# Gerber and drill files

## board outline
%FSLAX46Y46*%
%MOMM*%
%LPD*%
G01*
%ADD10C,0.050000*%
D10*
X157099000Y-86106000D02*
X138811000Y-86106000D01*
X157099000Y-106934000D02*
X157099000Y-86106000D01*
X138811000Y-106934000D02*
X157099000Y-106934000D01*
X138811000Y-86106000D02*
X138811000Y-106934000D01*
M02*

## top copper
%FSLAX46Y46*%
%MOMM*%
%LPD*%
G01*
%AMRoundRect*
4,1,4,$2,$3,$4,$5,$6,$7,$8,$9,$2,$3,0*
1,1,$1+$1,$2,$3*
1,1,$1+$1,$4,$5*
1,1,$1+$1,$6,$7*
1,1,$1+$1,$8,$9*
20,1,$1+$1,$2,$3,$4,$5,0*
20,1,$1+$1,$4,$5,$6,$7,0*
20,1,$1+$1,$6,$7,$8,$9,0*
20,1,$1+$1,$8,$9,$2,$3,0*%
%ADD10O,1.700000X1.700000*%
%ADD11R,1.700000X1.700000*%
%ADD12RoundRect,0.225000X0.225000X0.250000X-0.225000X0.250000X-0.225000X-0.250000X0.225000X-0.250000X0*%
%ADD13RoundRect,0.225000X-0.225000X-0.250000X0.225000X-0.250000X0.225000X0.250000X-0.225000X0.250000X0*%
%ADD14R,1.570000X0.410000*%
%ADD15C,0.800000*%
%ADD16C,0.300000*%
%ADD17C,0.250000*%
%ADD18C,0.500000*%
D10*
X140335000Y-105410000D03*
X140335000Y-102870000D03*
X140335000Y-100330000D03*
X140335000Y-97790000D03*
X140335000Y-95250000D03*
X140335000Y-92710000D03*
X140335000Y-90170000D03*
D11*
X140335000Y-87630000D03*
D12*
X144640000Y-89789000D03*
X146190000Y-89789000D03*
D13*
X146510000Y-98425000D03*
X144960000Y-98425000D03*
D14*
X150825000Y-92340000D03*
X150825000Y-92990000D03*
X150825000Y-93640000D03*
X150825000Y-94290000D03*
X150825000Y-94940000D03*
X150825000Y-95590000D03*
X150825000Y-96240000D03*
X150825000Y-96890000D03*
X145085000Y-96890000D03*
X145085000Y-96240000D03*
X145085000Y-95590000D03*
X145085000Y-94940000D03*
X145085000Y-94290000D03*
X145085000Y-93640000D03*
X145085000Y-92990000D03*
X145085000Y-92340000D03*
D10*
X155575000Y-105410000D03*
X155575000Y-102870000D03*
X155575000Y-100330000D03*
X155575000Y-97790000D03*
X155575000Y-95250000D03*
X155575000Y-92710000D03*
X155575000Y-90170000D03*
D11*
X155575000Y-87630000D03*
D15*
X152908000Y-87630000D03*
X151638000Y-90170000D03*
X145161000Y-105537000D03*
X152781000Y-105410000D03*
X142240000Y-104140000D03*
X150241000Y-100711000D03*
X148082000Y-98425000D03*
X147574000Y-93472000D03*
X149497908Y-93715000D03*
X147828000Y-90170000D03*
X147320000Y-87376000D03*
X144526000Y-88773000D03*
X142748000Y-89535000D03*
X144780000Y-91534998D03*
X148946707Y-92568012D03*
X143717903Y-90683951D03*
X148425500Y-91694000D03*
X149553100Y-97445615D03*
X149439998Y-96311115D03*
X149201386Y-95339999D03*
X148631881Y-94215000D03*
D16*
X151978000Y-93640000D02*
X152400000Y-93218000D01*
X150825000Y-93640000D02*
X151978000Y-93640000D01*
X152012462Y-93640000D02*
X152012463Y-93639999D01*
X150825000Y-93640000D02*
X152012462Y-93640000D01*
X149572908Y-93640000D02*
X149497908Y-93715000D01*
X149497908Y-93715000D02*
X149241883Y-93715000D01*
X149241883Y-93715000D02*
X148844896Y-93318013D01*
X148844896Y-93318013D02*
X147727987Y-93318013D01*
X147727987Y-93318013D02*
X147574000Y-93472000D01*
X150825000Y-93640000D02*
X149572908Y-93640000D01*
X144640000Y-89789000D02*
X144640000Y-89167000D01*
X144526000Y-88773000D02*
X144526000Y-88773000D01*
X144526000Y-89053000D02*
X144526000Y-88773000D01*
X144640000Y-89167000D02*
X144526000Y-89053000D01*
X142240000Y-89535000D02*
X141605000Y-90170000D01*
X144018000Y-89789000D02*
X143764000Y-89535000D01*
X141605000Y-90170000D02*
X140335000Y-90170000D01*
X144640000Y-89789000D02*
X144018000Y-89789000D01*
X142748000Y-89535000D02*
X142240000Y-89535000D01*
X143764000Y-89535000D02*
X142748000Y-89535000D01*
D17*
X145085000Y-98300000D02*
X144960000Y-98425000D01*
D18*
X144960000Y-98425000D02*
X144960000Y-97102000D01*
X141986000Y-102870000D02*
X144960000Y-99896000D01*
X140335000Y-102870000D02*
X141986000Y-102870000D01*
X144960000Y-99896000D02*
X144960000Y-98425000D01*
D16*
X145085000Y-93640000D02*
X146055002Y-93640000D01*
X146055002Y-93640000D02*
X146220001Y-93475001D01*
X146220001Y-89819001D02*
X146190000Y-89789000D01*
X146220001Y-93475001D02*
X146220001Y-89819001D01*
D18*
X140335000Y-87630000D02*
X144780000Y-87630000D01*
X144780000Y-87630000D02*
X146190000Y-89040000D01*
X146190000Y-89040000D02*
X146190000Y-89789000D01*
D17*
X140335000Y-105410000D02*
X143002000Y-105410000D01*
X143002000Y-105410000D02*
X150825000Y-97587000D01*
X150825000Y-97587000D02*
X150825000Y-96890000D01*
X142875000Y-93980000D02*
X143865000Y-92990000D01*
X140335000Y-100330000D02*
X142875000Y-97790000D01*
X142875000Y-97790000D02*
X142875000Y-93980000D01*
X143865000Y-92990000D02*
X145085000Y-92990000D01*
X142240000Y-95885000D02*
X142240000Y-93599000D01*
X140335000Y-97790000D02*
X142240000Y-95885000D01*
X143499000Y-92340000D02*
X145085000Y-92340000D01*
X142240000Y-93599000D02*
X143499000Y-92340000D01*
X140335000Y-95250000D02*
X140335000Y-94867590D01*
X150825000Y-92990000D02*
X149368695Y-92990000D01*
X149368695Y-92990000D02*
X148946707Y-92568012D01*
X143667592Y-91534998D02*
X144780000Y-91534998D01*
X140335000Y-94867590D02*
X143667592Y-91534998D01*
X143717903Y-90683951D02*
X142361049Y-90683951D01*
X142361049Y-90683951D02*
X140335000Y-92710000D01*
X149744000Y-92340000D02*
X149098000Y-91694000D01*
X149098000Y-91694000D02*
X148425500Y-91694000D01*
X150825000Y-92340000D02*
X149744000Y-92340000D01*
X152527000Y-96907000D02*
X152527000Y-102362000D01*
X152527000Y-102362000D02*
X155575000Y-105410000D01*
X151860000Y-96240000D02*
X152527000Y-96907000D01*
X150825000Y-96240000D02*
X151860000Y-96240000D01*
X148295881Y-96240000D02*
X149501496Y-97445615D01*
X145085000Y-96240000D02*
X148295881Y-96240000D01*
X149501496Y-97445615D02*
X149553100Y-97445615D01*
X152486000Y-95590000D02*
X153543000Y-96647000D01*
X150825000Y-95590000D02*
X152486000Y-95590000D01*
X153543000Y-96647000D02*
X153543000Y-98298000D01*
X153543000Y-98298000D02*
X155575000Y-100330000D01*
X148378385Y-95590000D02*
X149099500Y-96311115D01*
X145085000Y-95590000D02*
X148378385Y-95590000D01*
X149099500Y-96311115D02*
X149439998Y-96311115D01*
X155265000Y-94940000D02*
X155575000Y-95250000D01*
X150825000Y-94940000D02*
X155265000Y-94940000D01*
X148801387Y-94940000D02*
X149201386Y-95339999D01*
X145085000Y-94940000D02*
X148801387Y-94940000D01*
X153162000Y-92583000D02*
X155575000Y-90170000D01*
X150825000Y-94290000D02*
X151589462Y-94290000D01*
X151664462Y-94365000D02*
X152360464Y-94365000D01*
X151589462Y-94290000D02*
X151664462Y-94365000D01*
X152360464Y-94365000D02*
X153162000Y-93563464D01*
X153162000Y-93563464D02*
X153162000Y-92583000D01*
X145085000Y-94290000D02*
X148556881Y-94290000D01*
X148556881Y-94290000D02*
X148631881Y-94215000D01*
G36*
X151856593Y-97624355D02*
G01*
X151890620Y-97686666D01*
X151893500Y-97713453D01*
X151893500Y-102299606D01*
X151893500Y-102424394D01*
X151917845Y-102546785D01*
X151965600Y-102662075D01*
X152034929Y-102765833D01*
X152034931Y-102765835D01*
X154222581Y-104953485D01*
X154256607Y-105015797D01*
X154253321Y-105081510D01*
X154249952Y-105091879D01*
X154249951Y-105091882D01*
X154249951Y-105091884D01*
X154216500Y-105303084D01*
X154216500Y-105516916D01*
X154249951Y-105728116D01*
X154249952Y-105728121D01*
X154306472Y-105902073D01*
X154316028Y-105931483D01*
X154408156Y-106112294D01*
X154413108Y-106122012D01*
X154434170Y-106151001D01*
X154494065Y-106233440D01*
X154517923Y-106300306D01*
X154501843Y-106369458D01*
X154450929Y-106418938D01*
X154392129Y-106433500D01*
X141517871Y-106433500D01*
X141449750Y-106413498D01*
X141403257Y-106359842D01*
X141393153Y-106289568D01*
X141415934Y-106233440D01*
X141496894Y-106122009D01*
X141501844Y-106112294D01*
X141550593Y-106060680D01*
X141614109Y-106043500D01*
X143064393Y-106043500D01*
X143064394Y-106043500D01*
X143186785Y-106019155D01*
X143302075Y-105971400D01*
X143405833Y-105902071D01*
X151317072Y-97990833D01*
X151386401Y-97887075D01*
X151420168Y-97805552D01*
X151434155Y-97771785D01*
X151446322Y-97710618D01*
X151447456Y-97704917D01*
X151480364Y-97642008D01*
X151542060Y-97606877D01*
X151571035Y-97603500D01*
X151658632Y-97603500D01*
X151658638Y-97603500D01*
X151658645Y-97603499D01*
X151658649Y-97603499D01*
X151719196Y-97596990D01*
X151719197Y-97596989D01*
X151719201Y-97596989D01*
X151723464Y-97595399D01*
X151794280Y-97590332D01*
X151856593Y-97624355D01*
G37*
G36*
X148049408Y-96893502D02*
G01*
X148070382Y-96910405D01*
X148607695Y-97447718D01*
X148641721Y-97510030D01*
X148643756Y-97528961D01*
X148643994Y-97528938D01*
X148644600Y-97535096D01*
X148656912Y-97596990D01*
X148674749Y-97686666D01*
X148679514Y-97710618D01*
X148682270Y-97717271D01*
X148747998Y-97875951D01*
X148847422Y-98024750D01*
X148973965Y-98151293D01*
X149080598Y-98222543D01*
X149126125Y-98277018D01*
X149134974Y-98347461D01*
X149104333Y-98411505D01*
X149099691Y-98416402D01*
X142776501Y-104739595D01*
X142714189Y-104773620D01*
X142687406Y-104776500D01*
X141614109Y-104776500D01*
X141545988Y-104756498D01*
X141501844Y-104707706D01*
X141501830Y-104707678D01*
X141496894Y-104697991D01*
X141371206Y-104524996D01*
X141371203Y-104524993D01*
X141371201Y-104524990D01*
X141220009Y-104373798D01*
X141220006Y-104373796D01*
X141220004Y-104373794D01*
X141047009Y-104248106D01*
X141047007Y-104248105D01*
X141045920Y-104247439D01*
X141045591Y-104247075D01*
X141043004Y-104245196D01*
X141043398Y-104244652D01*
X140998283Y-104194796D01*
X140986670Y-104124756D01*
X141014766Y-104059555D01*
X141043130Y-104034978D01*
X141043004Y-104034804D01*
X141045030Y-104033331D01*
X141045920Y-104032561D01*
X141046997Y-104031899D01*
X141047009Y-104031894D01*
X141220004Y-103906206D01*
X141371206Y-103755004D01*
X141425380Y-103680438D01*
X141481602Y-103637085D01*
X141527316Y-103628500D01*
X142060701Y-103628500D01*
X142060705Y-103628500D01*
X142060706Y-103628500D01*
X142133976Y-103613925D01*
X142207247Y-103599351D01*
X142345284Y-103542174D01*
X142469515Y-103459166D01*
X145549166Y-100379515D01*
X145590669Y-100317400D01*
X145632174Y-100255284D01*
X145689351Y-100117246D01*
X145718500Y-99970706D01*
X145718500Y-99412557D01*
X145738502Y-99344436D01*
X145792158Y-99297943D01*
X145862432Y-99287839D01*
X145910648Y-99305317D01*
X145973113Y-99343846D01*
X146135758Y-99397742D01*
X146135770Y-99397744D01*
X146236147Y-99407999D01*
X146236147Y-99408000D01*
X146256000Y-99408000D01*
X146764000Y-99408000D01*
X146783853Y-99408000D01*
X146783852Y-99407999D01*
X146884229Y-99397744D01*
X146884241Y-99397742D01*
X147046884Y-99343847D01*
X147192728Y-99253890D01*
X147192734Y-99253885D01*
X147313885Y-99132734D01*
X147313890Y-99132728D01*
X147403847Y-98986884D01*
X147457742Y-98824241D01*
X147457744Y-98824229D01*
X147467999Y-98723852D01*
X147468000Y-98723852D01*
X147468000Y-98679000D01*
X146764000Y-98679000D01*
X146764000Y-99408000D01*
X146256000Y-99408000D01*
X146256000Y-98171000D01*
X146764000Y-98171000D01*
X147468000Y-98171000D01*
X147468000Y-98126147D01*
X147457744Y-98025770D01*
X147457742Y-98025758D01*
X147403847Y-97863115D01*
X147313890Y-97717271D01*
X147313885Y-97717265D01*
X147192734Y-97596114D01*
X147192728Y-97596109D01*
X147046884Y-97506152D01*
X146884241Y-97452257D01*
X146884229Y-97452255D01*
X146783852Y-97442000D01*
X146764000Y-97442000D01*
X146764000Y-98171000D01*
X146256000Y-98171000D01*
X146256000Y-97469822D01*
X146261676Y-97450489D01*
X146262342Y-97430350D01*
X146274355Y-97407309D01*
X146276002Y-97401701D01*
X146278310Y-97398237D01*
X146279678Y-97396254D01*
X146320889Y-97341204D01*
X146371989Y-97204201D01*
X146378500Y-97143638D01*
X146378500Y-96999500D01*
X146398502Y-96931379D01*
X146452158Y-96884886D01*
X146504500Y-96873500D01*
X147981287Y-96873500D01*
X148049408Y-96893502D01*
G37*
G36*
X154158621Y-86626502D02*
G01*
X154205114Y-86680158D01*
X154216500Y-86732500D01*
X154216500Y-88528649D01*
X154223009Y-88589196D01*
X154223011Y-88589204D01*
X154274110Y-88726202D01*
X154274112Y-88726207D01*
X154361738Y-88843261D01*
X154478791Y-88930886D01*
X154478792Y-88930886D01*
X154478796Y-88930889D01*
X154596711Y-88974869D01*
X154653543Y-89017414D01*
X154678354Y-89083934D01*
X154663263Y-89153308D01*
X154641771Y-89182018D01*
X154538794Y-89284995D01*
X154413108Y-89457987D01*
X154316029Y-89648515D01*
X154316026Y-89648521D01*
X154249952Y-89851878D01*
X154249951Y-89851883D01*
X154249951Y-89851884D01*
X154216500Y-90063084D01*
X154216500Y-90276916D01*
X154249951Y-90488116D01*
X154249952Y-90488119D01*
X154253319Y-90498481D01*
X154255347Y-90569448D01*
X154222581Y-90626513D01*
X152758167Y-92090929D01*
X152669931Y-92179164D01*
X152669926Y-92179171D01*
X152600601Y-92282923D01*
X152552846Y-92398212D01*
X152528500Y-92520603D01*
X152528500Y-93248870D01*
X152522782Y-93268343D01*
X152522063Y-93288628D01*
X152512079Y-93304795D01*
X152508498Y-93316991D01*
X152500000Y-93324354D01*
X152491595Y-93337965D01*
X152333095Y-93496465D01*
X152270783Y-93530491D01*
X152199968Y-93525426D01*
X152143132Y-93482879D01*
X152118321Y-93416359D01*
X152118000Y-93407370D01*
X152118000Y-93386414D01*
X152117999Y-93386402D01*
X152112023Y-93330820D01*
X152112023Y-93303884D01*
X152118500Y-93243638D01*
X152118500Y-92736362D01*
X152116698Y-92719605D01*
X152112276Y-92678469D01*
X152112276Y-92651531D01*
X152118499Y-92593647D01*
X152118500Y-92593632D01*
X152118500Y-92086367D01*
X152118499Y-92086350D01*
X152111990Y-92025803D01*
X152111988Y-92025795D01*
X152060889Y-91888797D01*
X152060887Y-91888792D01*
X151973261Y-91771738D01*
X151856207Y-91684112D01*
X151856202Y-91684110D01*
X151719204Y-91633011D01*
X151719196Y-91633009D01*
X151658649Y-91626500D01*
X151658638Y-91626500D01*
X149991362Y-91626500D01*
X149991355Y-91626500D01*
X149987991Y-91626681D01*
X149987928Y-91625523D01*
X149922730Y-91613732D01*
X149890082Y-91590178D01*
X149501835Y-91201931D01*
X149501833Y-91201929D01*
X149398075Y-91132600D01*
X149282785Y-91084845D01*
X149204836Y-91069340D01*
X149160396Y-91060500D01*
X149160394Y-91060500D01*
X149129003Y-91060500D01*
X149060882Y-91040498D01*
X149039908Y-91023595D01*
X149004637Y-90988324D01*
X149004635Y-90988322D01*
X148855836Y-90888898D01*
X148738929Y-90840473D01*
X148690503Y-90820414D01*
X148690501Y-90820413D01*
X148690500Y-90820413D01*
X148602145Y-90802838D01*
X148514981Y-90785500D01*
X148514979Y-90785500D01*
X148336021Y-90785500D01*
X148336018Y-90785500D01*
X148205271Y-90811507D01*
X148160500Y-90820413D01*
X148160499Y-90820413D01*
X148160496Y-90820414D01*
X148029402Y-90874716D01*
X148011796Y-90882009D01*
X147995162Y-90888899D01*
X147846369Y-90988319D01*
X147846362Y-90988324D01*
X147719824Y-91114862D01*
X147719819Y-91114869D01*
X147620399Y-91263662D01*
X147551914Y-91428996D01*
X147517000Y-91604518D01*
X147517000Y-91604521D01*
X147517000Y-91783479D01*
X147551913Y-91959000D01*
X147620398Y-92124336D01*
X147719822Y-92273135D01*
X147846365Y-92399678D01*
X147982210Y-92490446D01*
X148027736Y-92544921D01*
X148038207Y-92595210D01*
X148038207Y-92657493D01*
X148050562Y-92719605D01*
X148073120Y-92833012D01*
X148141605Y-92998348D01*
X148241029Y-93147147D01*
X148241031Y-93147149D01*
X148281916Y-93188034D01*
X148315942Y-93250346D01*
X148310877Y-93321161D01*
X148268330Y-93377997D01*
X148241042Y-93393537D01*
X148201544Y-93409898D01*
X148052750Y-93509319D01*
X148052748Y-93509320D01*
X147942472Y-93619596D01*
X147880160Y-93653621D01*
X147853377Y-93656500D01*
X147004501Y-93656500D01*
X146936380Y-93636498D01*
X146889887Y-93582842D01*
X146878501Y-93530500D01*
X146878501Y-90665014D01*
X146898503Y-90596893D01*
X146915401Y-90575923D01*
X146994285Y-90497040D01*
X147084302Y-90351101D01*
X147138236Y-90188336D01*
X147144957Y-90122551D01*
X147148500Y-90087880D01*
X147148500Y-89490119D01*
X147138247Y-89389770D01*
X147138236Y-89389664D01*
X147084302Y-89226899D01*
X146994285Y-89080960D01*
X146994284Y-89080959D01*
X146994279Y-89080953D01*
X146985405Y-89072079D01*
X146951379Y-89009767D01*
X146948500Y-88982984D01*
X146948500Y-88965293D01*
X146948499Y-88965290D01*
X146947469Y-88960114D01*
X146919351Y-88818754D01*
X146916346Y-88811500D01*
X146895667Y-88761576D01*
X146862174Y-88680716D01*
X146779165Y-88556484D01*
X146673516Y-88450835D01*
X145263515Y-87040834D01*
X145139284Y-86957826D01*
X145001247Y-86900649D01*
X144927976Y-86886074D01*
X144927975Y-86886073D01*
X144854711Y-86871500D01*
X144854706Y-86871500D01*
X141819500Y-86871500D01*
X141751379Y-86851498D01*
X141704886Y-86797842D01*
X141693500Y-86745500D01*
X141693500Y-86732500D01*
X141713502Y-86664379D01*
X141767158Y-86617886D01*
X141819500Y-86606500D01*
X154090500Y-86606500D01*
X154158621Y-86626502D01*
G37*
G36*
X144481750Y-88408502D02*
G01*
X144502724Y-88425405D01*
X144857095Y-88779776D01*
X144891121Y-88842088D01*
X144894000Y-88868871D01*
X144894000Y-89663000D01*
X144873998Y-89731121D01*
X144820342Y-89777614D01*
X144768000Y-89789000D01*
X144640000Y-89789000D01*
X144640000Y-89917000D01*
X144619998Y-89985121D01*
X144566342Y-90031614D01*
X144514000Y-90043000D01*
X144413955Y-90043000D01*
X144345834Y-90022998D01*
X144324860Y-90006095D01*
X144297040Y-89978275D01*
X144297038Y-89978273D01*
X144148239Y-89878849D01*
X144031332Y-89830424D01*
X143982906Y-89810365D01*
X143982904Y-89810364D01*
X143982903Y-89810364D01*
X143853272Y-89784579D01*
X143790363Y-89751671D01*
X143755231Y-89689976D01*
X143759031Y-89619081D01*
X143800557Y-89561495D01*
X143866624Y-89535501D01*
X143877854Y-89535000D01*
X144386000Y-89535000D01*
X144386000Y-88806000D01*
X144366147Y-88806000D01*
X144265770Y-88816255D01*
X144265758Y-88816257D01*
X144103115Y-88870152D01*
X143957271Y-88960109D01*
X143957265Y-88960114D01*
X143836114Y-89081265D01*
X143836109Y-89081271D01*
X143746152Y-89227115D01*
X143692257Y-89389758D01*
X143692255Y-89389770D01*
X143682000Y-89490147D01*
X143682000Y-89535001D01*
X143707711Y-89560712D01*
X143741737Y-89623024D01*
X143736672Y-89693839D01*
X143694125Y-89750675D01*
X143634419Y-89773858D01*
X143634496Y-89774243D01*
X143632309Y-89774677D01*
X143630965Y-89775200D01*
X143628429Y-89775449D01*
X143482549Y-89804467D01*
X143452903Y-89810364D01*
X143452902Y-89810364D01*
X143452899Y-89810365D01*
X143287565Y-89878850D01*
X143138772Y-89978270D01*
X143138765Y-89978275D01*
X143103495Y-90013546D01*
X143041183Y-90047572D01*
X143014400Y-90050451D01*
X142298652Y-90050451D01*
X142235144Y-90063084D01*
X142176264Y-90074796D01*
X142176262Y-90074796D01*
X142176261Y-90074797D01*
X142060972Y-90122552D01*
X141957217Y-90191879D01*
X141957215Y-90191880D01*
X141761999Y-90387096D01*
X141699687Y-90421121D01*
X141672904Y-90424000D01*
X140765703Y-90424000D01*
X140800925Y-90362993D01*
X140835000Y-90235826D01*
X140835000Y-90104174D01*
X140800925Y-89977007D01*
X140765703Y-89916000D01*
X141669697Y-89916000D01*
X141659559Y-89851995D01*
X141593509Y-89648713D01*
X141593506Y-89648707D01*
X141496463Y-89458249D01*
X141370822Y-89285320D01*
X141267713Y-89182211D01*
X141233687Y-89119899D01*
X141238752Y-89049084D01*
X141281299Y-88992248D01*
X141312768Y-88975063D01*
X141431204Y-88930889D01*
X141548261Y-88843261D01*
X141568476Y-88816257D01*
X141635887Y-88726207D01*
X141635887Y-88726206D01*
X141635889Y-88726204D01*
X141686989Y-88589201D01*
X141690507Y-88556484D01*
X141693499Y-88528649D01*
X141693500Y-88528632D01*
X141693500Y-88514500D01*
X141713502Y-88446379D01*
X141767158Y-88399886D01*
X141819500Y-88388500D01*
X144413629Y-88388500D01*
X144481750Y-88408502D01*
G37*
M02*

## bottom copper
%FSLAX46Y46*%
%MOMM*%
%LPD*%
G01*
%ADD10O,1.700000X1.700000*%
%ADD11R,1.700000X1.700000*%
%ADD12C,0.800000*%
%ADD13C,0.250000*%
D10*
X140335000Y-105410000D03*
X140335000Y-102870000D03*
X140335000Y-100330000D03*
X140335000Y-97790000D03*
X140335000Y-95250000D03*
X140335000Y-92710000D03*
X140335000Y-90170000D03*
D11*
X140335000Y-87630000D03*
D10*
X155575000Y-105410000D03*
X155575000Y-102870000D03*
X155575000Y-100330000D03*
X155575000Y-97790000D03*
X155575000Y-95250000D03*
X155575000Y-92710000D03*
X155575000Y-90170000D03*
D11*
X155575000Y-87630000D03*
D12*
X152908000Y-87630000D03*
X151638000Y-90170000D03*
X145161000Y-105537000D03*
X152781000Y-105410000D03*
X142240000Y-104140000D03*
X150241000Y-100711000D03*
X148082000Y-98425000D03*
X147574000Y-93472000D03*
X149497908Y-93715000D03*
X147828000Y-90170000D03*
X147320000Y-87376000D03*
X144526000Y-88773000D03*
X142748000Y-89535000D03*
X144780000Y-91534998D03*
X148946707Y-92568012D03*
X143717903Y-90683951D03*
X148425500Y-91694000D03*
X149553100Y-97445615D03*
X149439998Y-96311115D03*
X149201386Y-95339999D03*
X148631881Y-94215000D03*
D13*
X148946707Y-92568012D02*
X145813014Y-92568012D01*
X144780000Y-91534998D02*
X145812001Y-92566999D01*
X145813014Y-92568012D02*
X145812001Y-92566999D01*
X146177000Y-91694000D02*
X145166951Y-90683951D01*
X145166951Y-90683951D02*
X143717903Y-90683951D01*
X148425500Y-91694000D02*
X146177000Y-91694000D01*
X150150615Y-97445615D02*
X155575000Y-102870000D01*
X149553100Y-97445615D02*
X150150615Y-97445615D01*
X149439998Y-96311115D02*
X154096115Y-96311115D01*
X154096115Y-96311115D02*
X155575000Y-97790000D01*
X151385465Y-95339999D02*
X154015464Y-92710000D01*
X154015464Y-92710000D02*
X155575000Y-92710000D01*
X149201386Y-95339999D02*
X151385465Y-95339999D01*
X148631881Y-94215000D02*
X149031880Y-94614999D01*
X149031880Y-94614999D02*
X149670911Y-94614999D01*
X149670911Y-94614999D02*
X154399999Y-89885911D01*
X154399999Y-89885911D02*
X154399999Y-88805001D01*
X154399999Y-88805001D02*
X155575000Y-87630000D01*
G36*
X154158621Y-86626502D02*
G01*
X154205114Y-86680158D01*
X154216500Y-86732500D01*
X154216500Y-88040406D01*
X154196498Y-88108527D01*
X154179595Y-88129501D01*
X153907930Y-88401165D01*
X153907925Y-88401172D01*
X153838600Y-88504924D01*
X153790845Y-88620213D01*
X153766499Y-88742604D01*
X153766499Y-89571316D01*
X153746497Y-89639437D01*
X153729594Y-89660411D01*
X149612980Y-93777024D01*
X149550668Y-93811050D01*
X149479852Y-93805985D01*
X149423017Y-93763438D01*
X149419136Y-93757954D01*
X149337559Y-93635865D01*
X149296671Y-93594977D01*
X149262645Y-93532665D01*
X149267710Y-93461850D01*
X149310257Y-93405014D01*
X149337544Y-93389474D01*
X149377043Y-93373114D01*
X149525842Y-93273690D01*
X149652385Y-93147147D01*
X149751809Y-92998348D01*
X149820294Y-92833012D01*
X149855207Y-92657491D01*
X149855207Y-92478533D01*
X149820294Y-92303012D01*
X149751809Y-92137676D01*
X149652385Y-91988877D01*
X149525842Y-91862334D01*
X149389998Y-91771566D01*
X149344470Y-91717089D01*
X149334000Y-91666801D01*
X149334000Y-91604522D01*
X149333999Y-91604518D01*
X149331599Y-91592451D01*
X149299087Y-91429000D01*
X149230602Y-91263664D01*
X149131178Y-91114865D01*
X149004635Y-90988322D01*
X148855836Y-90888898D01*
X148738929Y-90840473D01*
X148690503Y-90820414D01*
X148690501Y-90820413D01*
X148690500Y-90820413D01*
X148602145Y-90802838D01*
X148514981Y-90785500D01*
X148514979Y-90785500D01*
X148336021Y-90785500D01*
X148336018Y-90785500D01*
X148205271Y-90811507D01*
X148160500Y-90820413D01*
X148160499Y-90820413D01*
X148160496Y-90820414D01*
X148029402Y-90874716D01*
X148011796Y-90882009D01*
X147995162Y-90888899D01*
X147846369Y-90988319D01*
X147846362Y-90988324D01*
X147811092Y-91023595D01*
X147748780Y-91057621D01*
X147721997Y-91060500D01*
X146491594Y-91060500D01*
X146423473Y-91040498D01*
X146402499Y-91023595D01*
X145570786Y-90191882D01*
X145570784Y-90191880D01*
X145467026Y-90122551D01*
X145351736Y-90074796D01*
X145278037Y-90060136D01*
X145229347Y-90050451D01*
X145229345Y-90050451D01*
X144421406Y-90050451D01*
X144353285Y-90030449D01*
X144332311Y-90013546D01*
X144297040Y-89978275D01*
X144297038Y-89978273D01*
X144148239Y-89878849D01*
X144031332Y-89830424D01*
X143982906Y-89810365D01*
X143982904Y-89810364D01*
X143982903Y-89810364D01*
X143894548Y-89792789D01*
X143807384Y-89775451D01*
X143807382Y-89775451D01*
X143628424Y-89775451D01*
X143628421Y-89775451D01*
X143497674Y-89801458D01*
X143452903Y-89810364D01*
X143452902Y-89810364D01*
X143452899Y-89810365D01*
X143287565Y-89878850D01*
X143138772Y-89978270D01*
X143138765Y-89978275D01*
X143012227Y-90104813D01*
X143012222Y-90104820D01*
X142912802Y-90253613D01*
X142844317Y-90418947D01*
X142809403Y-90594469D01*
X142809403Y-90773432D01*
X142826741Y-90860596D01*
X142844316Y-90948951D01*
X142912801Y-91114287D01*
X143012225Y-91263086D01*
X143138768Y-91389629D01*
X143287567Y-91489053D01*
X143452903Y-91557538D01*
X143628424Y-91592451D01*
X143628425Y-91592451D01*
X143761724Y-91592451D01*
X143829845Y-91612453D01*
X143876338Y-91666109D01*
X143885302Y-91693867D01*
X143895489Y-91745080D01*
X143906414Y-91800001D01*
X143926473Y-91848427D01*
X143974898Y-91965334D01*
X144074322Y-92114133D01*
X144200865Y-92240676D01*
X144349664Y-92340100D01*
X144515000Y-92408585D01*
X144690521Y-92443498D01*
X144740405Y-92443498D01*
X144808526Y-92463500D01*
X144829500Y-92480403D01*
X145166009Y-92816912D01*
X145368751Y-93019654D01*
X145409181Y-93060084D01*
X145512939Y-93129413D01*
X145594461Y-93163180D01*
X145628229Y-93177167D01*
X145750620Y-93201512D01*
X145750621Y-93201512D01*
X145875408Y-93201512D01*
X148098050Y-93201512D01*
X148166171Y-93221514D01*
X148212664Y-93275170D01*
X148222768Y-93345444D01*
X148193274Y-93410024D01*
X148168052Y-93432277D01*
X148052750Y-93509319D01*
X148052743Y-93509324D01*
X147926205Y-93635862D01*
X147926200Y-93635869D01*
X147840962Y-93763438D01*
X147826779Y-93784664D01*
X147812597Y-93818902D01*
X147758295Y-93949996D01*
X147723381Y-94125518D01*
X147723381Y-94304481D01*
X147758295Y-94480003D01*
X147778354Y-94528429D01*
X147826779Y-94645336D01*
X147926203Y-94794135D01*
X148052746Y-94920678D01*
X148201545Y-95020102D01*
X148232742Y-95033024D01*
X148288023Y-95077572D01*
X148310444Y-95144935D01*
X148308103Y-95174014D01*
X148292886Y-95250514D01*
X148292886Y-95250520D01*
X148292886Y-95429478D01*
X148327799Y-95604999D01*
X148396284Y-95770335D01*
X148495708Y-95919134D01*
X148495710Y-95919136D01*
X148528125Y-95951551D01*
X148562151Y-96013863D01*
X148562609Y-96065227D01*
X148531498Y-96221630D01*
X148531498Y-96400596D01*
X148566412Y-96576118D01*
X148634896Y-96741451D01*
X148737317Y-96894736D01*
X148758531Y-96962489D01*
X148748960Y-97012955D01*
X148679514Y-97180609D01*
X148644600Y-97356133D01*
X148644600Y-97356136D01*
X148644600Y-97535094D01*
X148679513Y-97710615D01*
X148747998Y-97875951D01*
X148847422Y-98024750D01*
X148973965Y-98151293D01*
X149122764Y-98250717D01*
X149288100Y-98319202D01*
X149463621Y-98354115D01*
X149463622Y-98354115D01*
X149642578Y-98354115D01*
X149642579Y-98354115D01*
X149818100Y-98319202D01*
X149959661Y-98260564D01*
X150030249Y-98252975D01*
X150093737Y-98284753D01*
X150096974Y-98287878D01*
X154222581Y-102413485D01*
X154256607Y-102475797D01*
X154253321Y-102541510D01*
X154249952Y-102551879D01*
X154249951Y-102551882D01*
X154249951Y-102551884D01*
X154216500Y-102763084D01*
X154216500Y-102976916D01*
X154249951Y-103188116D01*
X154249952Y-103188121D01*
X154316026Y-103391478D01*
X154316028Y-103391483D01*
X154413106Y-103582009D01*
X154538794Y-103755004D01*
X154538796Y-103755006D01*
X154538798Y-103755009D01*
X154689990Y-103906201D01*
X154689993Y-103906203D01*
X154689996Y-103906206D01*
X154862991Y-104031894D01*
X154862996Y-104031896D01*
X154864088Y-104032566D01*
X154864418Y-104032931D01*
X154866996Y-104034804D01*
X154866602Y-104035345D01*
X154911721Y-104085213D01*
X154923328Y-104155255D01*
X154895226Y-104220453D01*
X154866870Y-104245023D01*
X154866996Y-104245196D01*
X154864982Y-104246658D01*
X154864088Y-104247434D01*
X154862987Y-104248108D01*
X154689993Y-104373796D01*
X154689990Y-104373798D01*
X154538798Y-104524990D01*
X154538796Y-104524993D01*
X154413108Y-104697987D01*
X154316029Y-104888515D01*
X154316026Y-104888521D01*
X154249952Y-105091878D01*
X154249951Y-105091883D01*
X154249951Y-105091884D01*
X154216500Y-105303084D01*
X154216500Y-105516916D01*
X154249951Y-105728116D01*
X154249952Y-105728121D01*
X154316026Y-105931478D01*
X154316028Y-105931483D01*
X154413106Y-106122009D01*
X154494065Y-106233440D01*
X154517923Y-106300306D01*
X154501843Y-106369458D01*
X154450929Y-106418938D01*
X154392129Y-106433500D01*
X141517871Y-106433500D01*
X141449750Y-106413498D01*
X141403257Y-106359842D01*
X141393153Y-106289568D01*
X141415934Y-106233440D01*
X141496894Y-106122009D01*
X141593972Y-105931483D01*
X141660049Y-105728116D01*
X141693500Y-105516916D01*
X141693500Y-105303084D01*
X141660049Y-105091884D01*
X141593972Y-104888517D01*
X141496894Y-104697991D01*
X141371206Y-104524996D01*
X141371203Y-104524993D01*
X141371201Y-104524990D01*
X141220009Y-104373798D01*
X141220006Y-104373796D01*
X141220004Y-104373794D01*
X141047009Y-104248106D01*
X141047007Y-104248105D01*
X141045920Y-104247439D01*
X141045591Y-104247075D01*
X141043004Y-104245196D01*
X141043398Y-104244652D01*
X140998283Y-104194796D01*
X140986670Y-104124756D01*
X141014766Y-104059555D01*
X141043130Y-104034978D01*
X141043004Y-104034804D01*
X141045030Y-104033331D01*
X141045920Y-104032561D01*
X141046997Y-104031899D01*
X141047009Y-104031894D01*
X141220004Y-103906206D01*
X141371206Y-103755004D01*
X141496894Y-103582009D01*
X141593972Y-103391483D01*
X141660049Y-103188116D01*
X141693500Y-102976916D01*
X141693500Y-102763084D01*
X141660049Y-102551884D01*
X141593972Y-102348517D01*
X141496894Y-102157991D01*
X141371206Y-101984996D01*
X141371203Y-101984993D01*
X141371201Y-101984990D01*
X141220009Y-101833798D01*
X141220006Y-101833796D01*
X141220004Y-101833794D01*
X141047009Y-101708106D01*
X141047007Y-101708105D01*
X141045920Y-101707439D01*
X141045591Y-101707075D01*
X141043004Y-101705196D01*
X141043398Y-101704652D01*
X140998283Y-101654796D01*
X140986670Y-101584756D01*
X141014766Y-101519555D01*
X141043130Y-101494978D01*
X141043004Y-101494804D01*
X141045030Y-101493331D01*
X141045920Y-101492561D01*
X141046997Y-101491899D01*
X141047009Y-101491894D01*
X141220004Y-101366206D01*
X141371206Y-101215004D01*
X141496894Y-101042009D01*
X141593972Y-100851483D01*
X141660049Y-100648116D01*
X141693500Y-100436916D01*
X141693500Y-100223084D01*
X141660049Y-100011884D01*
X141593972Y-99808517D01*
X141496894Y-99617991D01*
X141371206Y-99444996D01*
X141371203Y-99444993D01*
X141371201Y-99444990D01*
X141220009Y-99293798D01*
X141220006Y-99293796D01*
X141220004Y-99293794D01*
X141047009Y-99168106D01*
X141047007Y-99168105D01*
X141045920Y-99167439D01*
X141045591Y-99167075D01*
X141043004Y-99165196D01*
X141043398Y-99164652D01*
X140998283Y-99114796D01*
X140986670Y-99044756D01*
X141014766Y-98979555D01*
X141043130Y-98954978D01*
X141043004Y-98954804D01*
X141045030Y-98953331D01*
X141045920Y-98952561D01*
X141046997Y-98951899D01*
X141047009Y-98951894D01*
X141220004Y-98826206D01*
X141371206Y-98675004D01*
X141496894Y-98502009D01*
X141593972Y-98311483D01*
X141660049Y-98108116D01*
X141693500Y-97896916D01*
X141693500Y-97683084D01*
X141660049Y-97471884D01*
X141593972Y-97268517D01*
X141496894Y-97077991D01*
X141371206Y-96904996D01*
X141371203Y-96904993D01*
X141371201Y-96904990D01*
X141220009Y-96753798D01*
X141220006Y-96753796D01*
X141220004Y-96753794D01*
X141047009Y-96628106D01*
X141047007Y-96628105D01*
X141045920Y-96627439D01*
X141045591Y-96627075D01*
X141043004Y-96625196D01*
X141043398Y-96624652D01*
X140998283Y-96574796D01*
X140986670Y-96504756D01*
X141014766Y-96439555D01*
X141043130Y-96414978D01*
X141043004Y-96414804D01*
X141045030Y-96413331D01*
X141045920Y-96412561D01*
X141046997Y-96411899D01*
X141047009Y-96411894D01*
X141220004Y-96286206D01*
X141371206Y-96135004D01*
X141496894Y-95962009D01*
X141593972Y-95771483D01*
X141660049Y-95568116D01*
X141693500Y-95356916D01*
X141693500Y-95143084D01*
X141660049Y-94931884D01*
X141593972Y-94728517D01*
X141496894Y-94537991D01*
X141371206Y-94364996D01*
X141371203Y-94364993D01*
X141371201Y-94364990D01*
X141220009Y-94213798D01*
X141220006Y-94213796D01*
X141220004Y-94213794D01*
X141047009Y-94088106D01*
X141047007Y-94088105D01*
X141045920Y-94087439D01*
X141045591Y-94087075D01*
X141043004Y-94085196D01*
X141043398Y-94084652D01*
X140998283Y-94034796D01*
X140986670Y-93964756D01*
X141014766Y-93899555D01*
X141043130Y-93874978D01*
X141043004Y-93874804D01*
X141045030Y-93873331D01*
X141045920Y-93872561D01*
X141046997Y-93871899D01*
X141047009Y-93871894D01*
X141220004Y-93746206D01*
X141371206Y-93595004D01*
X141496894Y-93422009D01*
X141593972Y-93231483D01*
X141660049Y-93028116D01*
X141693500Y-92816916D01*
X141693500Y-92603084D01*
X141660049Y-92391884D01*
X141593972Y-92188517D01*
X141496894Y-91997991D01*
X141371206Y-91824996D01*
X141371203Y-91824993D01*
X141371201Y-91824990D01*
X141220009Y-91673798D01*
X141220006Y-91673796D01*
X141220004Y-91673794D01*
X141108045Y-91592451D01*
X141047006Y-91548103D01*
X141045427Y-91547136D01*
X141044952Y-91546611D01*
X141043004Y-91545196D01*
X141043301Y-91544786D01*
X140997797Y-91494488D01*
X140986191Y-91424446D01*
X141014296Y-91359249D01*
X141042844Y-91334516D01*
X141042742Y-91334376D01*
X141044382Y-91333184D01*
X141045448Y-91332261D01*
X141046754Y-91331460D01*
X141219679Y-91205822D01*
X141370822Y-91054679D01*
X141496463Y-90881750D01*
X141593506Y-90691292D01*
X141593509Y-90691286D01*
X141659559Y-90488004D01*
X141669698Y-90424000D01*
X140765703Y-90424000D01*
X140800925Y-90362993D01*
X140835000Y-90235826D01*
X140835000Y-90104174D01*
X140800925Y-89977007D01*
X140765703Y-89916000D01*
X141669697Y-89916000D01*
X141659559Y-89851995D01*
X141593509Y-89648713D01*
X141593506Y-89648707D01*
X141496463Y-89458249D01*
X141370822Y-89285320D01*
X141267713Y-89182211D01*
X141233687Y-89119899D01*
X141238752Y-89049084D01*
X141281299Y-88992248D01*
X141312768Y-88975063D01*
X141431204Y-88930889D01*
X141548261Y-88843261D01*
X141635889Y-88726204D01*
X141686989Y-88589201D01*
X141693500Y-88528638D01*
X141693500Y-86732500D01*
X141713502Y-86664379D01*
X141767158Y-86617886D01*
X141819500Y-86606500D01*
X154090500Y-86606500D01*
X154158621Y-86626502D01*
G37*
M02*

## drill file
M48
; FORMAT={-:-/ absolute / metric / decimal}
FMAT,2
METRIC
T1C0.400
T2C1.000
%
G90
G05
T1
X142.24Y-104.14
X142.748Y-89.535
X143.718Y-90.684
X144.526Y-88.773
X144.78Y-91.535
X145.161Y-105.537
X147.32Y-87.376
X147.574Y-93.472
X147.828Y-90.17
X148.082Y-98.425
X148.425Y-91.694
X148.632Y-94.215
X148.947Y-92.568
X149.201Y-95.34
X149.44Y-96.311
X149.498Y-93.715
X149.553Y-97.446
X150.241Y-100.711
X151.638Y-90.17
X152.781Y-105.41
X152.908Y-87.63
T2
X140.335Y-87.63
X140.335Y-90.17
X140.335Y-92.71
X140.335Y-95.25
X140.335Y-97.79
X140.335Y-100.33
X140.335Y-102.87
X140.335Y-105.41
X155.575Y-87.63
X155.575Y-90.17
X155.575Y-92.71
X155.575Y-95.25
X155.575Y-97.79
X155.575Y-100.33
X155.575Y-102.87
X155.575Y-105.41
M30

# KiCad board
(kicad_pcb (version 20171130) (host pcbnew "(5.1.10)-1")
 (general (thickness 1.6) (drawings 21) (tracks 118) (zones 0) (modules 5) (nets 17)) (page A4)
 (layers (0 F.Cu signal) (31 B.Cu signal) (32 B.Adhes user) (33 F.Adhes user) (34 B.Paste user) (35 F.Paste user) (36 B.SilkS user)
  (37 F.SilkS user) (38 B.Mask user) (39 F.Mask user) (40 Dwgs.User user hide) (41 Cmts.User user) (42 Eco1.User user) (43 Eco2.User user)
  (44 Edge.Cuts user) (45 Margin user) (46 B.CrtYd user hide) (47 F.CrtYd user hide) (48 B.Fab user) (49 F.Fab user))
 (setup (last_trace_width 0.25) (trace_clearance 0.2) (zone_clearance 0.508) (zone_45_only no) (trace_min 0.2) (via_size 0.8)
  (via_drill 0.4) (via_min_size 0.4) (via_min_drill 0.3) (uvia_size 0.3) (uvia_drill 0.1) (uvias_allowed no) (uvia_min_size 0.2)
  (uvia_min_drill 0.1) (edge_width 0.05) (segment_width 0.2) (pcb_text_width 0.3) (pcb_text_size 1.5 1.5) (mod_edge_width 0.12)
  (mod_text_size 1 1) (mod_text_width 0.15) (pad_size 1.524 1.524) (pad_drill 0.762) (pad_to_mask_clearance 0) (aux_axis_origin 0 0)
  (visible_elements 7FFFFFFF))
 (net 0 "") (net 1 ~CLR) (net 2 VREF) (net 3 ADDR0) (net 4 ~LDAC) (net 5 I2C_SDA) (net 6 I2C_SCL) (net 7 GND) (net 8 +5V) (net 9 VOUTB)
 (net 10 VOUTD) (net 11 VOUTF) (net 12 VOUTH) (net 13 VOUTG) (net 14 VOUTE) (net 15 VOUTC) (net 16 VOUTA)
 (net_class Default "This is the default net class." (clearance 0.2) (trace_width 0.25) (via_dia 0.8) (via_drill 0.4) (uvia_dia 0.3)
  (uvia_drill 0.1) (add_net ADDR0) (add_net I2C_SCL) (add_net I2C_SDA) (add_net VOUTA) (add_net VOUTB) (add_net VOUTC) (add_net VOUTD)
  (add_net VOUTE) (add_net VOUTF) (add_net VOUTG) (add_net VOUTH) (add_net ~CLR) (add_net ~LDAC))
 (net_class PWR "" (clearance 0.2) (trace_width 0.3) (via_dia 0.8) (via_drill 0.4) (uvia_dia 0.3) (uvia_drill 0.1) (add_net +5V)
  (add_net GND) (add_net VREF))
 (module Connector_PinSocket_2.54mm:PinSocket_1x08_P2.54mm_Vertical (layer B.Cu) (at 140.335 87.63 180)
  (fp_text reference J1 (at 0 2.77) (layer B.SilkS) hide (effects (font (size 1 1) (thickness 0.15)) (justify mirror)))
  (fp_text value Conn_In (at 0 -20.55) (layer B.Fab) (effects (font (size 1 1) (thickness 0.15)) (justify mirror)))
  (pad 8 thru_hole oval (at 0 -17.78 180) (size 1.7 1.7) (drill 1) (layers *.Cu *.Mask) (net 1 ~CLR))
  (pad 7 thru_hole oval (at 0 -15.24 180) (size 1.7 1.7) (drill 1) (layers *.Cu *.Mask) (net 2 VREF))
  (pad 6 thru_hole oval (at 0 -12.7 180) (size 1.7 1.7) (drill 1) (layers *.Cu *.Mask) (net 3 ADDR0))
  (pad 5 thru_hole oval (at 0 -10.16 180) (size 1.7 1.7) (drill 1) (layers *.Cu *.Mask) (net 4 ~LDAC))
  (pad 4 thru_hole oval (at 0 -7.62 180) (size 1.7 1.7) (drill 1) (layers *.Cu *.Mask) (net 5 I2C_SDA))
  (pad 3 thru_hole oval (at 0 -5.08 180) (size 1.7 1.7) (drill 1) (layers *.Cu *.Mask) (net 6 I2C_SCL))
  (pad 2 thru_hole oval (at 0 -2.54 180) (size 1.7 1.7) (drill 1) (layers *.Cu *.Mask) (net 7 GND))
  (pad 1 thru_hole rect (at 0 0 180) (size 1.7 1.7) (drill 1) (layers *.Cu *.Mask) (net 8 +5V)))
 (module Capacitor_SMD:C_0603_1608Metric (layer F.Cu) (at 145.415 89.789 180)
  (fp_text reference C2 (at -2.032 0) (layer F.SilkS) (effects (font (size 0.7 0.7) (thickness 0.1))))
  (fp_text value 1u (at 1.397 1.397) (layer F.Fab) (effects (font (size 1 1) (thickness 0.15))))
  (pad 2 smd roundrect (at 0.775 0 180) (size 0.9 0.95) (layers F.Cu F.Paste F.Mask) (roundrect_rratio 0.25) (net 7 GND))
  (pad 1 smd roundrect (at -0.775 0 180) (size 0.9 0.95) (layers F.Cu F.Paste F.Mask) (roundrect_rratio 0.25) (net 8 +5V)))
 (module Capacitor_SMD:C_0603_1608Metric (layer F.Cu) (at 145.735 98.425)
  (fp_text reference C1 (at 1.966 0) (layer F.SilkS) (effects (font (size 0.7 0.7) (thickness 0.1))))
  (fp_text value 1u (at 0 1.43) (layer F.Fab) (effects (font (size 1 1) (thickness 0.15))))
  (pad 2 smd roundrect (at 0.775 0) (size 0.9 0.95) (layers F.Cu F.Paste F.Mask) (roundrect_rratio 0.25) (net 7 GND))
  (pad 1 smd roundrect (at -0.775 0) (size 0.9 0.95) (layers F.Cu F.Paste F.Mask) (roundrect_rratio 0.25) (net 2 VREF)))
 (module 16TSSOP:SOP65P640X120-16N (layer F.Cu) (at 147.955 94.615)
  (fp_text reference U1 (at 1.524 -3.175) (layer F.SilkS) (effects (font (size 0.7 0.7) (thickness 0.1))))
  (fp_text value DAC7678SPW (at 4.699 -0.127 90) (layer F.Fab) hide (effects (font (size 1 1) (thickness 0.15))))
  (pad 16 smd rect (at 2.87 -2.275) (size 1.57 0.41) (layers F.Cu F.Paste F.Mask) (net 6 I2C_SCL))
  (pad 15 smd rect (at 2.87 -1.625) (size 1.57 0.41) (layers F.Cu F.Paste F.Mask) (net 5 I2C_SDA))
  (pad 14 smd rect (at 2.87 -0.975) (size 1.57 0.41) (layers F.Cu F.Paste F.Mask) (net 7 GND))
  (pad 13 smd rect (at 2.87 -0.325) (size 1.57 0.41) (layers F.Cu F.Paste F.Mask) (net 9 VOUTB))
  (pad 12 smd rect (at 2.87 0.325) (size 1.57 0.41) (layers F.Cu F.Paste F.Mask) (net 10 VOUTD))
  (pad 11 smd rect (at 2.87 0.975) (size 1.57 0.41) (layers F.Cu F.Paste F.Mask) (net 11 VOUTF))
  (pad 10 smd rect (at 2.87 1.625) (size 1.57 0.41) (layers F.Cu F.Paste F.Mask) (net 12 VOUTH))
  (pad 9 smd rect (at 2.87 2.275) (size 1.57 0.41) (layers F.Cu F.Paste F.Mask) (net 1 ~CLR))
  (pad 8 smd rect (at -2.87 2.275) (size 1.57 0.41) (layers F.Cu F.Paste F.Mask) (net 2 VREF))
  (pad 7 smd rect (at -2.87 1.625) (size 1.57 0.41) (layers F.Cu F.Paste F.Mask) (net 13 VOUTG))
  (pad 6 smd rect (at -2.87 0.975) (size 1.57 0.41) (layers F.Cu F.Paste F.Mask) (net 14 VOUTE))
  (pad 5 smd rect (at -2.87 0.325) (size 1.57 0.41) (layers F.Cu F.Paste F.Mask) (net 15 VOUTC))
  (pad 4 smd rect (at -2.87 -0.325) (size 1.57 0.41) (layers F.Cu F.Paste F.Mask) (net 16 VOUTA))
  (pad 3 smd rect (at -2.87 -0.975) (size 1.57 0.41) (layers F.Cu F.Paste F.Mask) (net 8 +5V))
  (pad 2 smd rect (at -2.87 -1.625) (size 1.57 0.41) (layers F.Cu F.Paste F.Mask) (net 3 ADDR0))
  (pad 1 smd rect (at -2.87 -2.275) (size 1.57 0.41) (layers F.Cu F.Paste F.Mask) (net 4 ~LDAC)))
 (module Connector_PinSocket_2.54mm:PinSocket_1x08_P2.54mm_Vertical (layer B.Cu) (at 155.575 87.63 180)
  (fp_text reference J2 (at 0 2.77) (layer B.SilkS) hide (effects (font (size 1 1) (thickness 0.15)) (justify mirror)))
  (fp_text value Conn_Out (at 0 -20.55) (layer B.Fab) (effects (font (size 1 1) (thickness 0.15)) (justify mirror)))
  (pad 8 thru_hole oval (at 0 -17.78 180) (size 1.7 1.7) (drill 1) (layers *.Cu *.Mask) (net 12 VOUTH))
  (pad 7 thru_hole oval (at 0 -15.24 180) (size 1.7 1.7) (drill 1) (layers *.Cu *.Mask) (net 13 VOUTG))
  (pad 6 thru_hole oval (at 0 -12.7 180) (size 1.7 1.7) (drill 1) (layers *.Cu *.Mask) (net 11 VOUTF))
  (pad 5 thru_hole oval (at 0 -10.16 180) (size 1.7 1.7) (drill 1) (layers *.Cu *.Mask) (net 14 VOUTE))
  (pad 4 thru_hole oval (at 0 -7.62 180) (size 1.7 1.7) (drill 1) (layers *.Cu *.Mask) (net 10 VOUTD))
  (pad 3 thru_hole oval (at 0 -5.08 180) (size 1.7 1.7) (drill 1) (layers *.Cu *.Mask) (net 15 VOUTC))
  (pad 2 thru_hole oval (at 0 -2.54 180) (size 1.7 1.7) (drill 1) (layers *.Cu *.Mask) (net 9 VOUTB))
  (pad 1 thru_hole rect (at 0 0 180) (size 1.7 1.7) (drill 1) (layers *.Cu *.Mask) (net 16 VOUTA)))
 (gr_line (start 157.099 86.106) (end 138.811 86.106) (layer Edge.Cuts) (width 0.05))
 (gr_line (start 157.099 106.934) (end 157.099 86.106) (layer Edge.Cuts) (width 0.05))
 (gr_line (start 138.811 106.934) (end 157.099 106.934) (layer Edge.Cuts) (width 0.05))
 (gr_line (start 138.811 86.106) (end 138.811 106.934) (layer Edge.Cuts) (width 0.05))
 (via (at 152.908 87.63) (size 0.8) (drill 0.4) (layers F.Cu B.Cu) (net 7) (status 1000000))
 (via (at 151.638 90.17) (size 0.8) (drill 0.4) (layers F.Cu B.Cu) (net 7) (status 1000000))
 (segment (start 151.978 93.64) (end 152.4 93.218) (width 0.3) (layer F.Cu) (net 7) (status 1000000))
 (segment (start 150.825 93.64) (end 151.978 93.64) (width 0.3) (layer F.Cu) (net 7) (status 1000000))
 (segment (start 152.012462 93.64) (end 152.012463 93.639999) (width 0.3) (layer F.Cu) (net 7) (status 1000000))
 (segment (start 150.825 93.64) (end 152.012462 93.64) (width 0.3) (layer F.Cu) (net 7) (status 1000000))
 (via (at 145.161 105.537) (size 0.8) (drill 0.4) (layers F.Cu B.Cu) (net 7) (status 1000000))
 (via (at 152.781 105.41) (size 0.8) (drill 0.4) (layers F.Cu B.Cu) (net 7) (status 1000000))
 (via (at 142.24 104.14) (size 0.8) (drill 0.4) (layers F.Cu B.Cu) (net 7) (status 1000000))
 (via (at 150.241 100.711) (size 0.8) (drill 0.4) (layers F.Cu B.Cu) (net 7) (status 1000000))
 (via (at 148.082 98.425) (size 0.8) (drill 0.4) (layers F.Cu B.Cu) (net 7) (status 1000000))
 (via (at 147.574 93.472) (size 0.8) (drill 0.4) (layers F.Cu B.Cu) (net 7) (status 1000000))
 (via (at 149.497908 93.715) (size 0.8) (drill 0.4) (layers F.Cu B.Cu) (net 7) (status 1000000))
 (segment (start 149.572908 93.64) (end 149.497908 93.715) (width 0.3) (layer F.Cu) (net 7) (status 1000000))
 (segment (start 149.497908 93.715) (end 149.241883 93.715) (width 0.3) (layer F.Cu) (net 7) (status 1000000))
 (segment (start 149.241883 93.715) (end 148.844896 93.318013) (width 0.3) (layer F.Cu) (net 7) (status 1000000))
 (segment (start 148.844896 93.318013) (end 147.727987 93.318013) (width 0.3) (layer F.Cu) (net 7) (status 1000000))
 (segment (start 147.727987 93.318013) (end 147.574 93.472) (width 0.3) (layer F.Cu) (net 7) (status 1000000))
 (segment (start 150.825 93.64) (end 149.572908 93.64) (width 0.3) (layer F.Cu) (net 7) (status 1000000))
 (via (at 147.828 90.17) (size 0.8) (drill 0.4) (layers F.Cu B.Cu) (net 7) (status 1000000))
 (via (at 147.32 87.376) (size 0.8) (drill 0.4) (layers F.Cu B.Cu) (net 7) (status 1000000))
 (segment (start 144.64 89.789) (end 144.64 89.167) (width 0.3) (layer F.Cu) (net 7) (status 1000000))
 (segment (start 144.526 88.773) (end 144.526 88.773) (width 0.3) (layer F.Cu) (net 7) (status 1000000))
 (segment (start 144.526 89.053) (end 144.526 88.773) (width 0.3) (layer F.Cu) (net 7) (status 1000000))
 (segment (start 144.64 89.167) (end 144.526 89.053) (width 0.3) (layer F.Cu) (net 7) (status 1000000))
 (via (at 144.526 88.773) (size 0.8) (drill 0.4) (layers F.Cu B.Cu) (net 7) (status 1000000))
 (via (at 142.748 89.535) (size 0.8) (drill 0.4) (layers F.Cu B.Cu) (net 7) (status 1000000))
 (segment (start 142.24 89.535) (end 141.605 90.17) (width 0.3) (layer F.Cu) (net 7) (status 1000000))
 (segment (start 144.018 89.789) (end 143.764 89.535) (width 0.3) (layer F.Cu) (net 7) (status 1000000))
 (segment (start 141.605 90.17) (end 140.335 90.17) (width 0.3) (layer F.Cu) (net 7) (status 1000000))
 (segment (start 144.64 89.789) (end 144.018 89.789) (width 0.3) (layer F.Cu) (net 7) (status 1000000))
 (segment (start 142.748 89.535) (end 142.24 89.535) (width 0.3) (layer F.Cu) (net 7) (status 1000000))
 (segment (start 143.764 89.535) (end 142.748 89.535) (width 0.3) (layer F.Cu) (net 7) (status 1000000))
 (segment (start 145.085 98.3) (end 144.96 98.425) (width 0.25) (layer F.Cu) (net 2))
 (segment (start 144.96 98.425) (end 144.96 97.102) (width 0.5) (layer F.Cu) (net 2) (status 1000000))
 (segment (start 141.986 102.87) (end 144.96 99.896) (width 0.5) (layer F.Cu) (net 2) (status 1000000))
 (segment (start 140.335 102.87) (end 141.986 102.87) (width 0.5) (layer F.Cu) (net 2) (status 1000000))
 (segment (start 144.96 99.896) (end 144.96 98.425) (width 0.5) (layer F.Cu) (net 2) (status 1000000))
 (segment (start 145.085 93.64) (end 146.055002 93.64) (width 0.3) (layer F.Cu) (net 8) (status 1000000))
 (segment (start 146.055002 93.64) (end 146.220001 93.475001) (width 0.3) (layer F.Cu) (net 8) (status 1000000))
 (segment (start 146.220001 89.819001) (end 146.19 89.789) (width 0.3) (layer F.Cu) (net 8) (status 1000000))
 (segment (start 146.220001 93.475001) (end 146.220001 89.819001) (width 0.3) (layer F.Cu) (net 8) (status 1000000))
 (segment (start 140.335 87.63) (end 144.78 87.63) (width 0.5) (layer F.Cu) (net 8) (status 1000000))
 (segment (start 144.78 87.63) (end 146.19 89.04) (width 0.5) (layer F.Cu) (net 8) (status 1000000))
 (segment (start 146.19 89.04) (end 146.19 89.789) (width 0.5) (layer F.Cu) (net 8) (status 1000000))
 (segment (start 140.335 105.41) (end 143.002 105.41) (width 0.25) (layer F.Cu) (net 1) (status 1000000))
 (segment (start 143.002 105.41) (end 150.825 97.587) (width 0.25) (layer F.Cu) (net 1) (status 1000000))
 (segment (start 150.825 97.587) (end 150.825 96.89) (width 0.25) (layer F.Cu) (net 1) (status 1000000))
 (segment (start 142.875 93.98) (end 143.865 92.99) (width 0.25) (layer F.Cu) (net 3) (status 1000000))
 (segment (start 140.335 100.33) (end 142.875 97.79) (width 0.25) (layer F.Cu) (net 3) (status 1000000))
 (segment (start 142.875 97.79) (end 142.875 93.98) (width 0.25) (layer F.Cu) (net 3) (status 1000000))
 (segment (start 143.865 92.99) (end 145.085 92.99) (width 0.25) (layer F.Cu) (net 3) (status 1000000))
 (segment (start 142.24 95.885) (end 142.24 93.599) (width 0.25) (layer F.Cu) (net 4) (status 1000000))
 (segment (start 140.335 97.79) (end 142.24 95.885) (width 0.25) (layer F.Cu) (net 4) (status 1000000))
 (segment (start 143.499 92.34) (end 145.085 92.34) (width 0.25) (layer F.Cu) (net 4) (status 1000000))
 (segment (start 142.24 93.599) (end 143.499 92.34) (width 0.25) (layer F.Cu) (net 4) (status 1000000))
 (via (at 144.78 91.534998) (size 0.8) (drill 0.4) (layers F.Cu B.Cu) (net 5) (status 1000000))
 (via (at 148.946707 92.568012) (size 0.8) (drill 0.4) (layers F.Cu B.Cu) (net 5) (status 1000000))
 (segment (start 148.946707 92.568012) (end 145.813014 92.568012) (width 0.25) (layer B.Cu) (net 5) (status 1000000))
 (segment (start 140.335 95.25) (end 140.335 94.86759) (width 0.25) (layer F.Cu) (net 5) (status 1000000))
 (segment (start 144.78 91.534998) (end 145.812001 92.566999) (width 0.25) (layer B.Cu) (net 5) (status 1000000))
 (segment (start 150.825 92.99) (end 149.368695 92.99) (width 0.25) (layer F.Cu) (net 5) (status 1000000))
 (segment (start 149.368695 92.99) (end 148.946707 92.568012) (width 0.25) (layer F.Cu) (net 5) (status 1000000))
 (segment (start 143.667592 91.534998) (end 144.78 91.534998) (width 0.25) (layer F.Cu) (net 5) (status 1000000))
 (segment (start 140.335 94.86759) (end 143.667592 91.534998) (width 0.25) (layer F.Cu) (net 5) (status 1000000))
 (segment (start 145.813014 92.568012) (end 145.812001 92.566999) (width 0.25) (layer B.Cu) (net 5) (status 1000000))
 (via (at 143.717903 90.683951) (size 0.8) (drill 0.4) (layers F.Cu B.Cu) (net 6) (status 1000000))
 (via (at 148.4255 91.694) (size 0.8) (drill 0.4) (layers F.Cu B.Cu) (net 6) (status 1000000))
 (segment (start 143.717903 90.683951) (end 142.361049 90.683951) (width 0.25) (layer F.Cu) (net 6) (status 1000000))
 (segment (start 146.177 91.694) (end 145.166951 90.683951) (width 0.25) (layer B.Cu) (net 6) (status 1000000))
 (segment (start 142.361049 90.683951) (end 140.335 92.71) (width 0.25) (layer F.Cu) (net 6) (status 1000000))
 (segment (start 149.744 92.34) (end 149.098 91.694) (width 0.25) (layer F.Cu) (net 6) (status 1000000))
 (segment (start 149.098 91.694) (end 148.4255 91.694) (width 0.25) (layer F.Cu) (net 6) (status 1000000))
 (segment (start 150.825 92.34) (end 149.744 92.34) (width 0.25) (layer F.Cu) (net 6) (status 1000000))
 (segment (start 145.166951 90.683951) (end 143.717903 90.683951) (width 0.25) (layer B.Cu) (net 6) (status 1000000))
 (segment (start 148.4255 91.694) (end 146.177 91.694) (width 0.25) (layer B.Cu) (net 6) (status 1000000))
 (segment (start 152.527 96.907) (end 152.527 102.362) (width 0.25) (layer F.Cu) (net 12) (status 1000000))
 (segment (start 152.527 102.362) (end 155.575 105.41) (width 0.25) (layer F.Cu) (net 12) (status 1000000))
 (segment (start 151.86 96.24) (end 152.527 96.907) (width 0.25) (layer F.Cu) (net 12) (status 1000000))
 (segment (start 150.825 96.24) (end 151.86 96.24) (width 0.25) (layer F.Cu) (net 12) (status 1000000))
 (via (at 149.5531 97.445615) (size 0.8) (drill 0.4) (layers F.Cu B.Cu) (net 13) (status 1000000))
 (segment (start 148.295881 96.24) (end 149.501496 97.445615) (width 0.25) (layer F.Cu) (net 13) (status 1000000))
 (segment (start 150.150615 97.445615) (end 155.575 102.87) (width 0.25) (layer B.Cu) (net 13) (status 1000000))
 (segment (start 149.5531 97.445615) (end 150.150615 97.445615) (width 0.25) (layer B.Cu) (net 13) (status 1000000))
 (segment (start 145.085 96.24) (end 148.295881 96.24) (width 0.25) (layer F.Cu) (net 13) (status 1000000))
 (segment (start 149.501496 97.445615) (end 149.5531 97.445615) (width 0.25) (layer F.Cu) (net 13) (status 1000000))
 (segment (start 152.486 95.59) (end 153.543 96.647) (width 0.25) (layer F.Cu) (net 11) (status 1000000))
 (segment (start 150.825 95.59) (end 152.486 95.59) (width 0.25) (layer F.Cu) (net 11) (status 1000000))
 (segment (start 153.543 96.647) (end 153.543 98.298) (width 0.25) (layer F.Cu) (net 11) (status 1000000))
 (segment (start 153.543 98.298) (end 155.575 100.33) (width 0.25) (layer F.Cu) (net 11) (status 1000000))
 (via (at 149.439998 96.311115) (size 0.8) (drill 0.4) (layers F.Cu B.Cu) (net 14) (status 1000000))
 (segment (start 149.439998 96.311115) (end 154.096115 96.311115) (width 0.25) (layer B.Cu) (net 14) (status 1000000))
 (segment (start 148.378385 95.59) (end 149.0995 96.311115) (width 0.25) (layer F.Cu) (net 14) (status 1000000))
 (segment (start 154.096115 96.311115) (end 155.575 97.79) (width 0.25) (layer B.Cu) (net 14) (status 1000000))
 (segment (start 145.085 95.59) (end 148.378385 95.59) (width 0.25) (layer F.Cu) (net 14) (status 1000000))
 (segment (start 149.0995 96.311115) (end 149.439998 96.311115) (width 0.25) (layer F.Cu) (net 14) (status 1000000))
 (segment (start 155.265 94.94) (end 155.575 95.25) (width 0.25) (layer F.Cu) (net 10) (status 1000000))
 (segment (start 150.825 94.94) (end 155.265 94.94) (width 0.25) (layer F.Cu) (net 10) (status 1000000))
 (via (at 149.201386 95.339999) (size 0.8) (drill 0.4) (layers F.Cu B.Cu) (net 15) (status 1000000))
 (segment (start 151.385465 95.339999) (end 154.015464 92.71) (width 0.25) (layer B.Cu) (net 15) (status 1000000))
 (segment (start 154.015464 92.71) (end 155.575 92.71) (width 0.25) (layer B.Cu) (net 15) (status 1000000))
 (segment (start 148.801387 94.94) (end 149.201386 95.339999) (width 0.25) (layer F.Cu) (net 15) (status 1000000))
 (segment (start 149.201386 95.339999) (end 151.385465 95.339999) (width 0.25) (layer B.Cu) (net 15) (status 1000000))
 (segment (start 145.085 94.94) (end 148.801387 94.94) (width 0.25) (layer F.Cu) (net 15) (status 1000000))
 (segment (start 153.162 92.583) (end 155.575 90.17) (width 0.25) (layer F.Cu) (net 9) (status 1000000))
 (segment (start 150.825 94.29) (end 151.589462 94.29) (width 0.25) (layer F.Cu) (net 9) (status 1000000))
 (segment (start 151.664462 94.365) (end 152.360464 94.365) (width 0.25) (layer F.Cu) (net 9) (status 1000000))
 (segment (start 151.589462 94.29) (end 151.664462 94.365) (width 0.25) (layer F.Cu) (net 9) (status 1000000))
 (segment (start 152.360464 94.365) (end 153.162 93.563464) (width 0.25) (layer F.Cu) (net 9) (status 1000000))
 (segment (start 153.162 93.563464) (end 153.162 92.583) (width 0.25) (layer F.Cu) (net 9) (status 1000000))
 (via (at 148.631881 94.215) (size 0.8) (drill 0.4) (layers F.Cu B.Cu) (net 16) (status 1000000))
 (segment (start 148.631881 94.215) (end 149.03188 94.614999) (width 0.25) (layer B.Cu) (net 16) (status 1000000))
 (segment (start 149.03188 94.614999) (end 149.670911 94.614999) (width 0.25) (layer B.Cu) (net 16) (status 1000000))
 (segment (start 149.670911 94.614999) (end 154.399999 89.885911) (width 0.25) (layer B.Cu) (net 16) (status 1000000))
 (segment (start 154.399999 89.885911) (end 154.399999 88.805001) (width 0.25) (layer B.Cu) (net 16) (status 1000000))
 (segment (start 154.399999 88.805001) (end 155.575 87.63) (width 0.25) (layer B.Cu) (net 16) (status 1000000))
 (segment (start 145.085 94.29) (end 148.556881 94.29) (width 0.25) (layer F.Cu) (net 16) (status 1000000))
 (segment (start 148.556881 94.29) (end 148.631881 94.215) (width 0.25) (layer F.Cu) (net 16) (status 1000000))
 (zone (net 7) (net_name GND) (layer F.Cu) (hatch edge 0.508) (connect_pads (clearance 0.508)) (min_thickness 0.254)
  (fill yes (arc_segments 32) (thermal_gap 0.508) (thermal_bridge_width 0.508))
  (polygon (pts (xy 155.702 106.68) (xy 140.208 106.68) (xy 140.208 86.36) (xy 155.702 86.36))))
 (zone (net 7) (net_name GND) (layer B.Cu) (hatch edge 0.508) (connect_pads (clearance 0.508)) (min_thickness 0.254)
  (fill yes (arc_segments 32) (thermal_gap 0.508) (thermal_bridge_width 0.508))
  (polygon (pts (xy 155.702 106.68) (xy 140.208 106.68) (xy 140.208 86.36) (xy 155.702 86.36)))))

